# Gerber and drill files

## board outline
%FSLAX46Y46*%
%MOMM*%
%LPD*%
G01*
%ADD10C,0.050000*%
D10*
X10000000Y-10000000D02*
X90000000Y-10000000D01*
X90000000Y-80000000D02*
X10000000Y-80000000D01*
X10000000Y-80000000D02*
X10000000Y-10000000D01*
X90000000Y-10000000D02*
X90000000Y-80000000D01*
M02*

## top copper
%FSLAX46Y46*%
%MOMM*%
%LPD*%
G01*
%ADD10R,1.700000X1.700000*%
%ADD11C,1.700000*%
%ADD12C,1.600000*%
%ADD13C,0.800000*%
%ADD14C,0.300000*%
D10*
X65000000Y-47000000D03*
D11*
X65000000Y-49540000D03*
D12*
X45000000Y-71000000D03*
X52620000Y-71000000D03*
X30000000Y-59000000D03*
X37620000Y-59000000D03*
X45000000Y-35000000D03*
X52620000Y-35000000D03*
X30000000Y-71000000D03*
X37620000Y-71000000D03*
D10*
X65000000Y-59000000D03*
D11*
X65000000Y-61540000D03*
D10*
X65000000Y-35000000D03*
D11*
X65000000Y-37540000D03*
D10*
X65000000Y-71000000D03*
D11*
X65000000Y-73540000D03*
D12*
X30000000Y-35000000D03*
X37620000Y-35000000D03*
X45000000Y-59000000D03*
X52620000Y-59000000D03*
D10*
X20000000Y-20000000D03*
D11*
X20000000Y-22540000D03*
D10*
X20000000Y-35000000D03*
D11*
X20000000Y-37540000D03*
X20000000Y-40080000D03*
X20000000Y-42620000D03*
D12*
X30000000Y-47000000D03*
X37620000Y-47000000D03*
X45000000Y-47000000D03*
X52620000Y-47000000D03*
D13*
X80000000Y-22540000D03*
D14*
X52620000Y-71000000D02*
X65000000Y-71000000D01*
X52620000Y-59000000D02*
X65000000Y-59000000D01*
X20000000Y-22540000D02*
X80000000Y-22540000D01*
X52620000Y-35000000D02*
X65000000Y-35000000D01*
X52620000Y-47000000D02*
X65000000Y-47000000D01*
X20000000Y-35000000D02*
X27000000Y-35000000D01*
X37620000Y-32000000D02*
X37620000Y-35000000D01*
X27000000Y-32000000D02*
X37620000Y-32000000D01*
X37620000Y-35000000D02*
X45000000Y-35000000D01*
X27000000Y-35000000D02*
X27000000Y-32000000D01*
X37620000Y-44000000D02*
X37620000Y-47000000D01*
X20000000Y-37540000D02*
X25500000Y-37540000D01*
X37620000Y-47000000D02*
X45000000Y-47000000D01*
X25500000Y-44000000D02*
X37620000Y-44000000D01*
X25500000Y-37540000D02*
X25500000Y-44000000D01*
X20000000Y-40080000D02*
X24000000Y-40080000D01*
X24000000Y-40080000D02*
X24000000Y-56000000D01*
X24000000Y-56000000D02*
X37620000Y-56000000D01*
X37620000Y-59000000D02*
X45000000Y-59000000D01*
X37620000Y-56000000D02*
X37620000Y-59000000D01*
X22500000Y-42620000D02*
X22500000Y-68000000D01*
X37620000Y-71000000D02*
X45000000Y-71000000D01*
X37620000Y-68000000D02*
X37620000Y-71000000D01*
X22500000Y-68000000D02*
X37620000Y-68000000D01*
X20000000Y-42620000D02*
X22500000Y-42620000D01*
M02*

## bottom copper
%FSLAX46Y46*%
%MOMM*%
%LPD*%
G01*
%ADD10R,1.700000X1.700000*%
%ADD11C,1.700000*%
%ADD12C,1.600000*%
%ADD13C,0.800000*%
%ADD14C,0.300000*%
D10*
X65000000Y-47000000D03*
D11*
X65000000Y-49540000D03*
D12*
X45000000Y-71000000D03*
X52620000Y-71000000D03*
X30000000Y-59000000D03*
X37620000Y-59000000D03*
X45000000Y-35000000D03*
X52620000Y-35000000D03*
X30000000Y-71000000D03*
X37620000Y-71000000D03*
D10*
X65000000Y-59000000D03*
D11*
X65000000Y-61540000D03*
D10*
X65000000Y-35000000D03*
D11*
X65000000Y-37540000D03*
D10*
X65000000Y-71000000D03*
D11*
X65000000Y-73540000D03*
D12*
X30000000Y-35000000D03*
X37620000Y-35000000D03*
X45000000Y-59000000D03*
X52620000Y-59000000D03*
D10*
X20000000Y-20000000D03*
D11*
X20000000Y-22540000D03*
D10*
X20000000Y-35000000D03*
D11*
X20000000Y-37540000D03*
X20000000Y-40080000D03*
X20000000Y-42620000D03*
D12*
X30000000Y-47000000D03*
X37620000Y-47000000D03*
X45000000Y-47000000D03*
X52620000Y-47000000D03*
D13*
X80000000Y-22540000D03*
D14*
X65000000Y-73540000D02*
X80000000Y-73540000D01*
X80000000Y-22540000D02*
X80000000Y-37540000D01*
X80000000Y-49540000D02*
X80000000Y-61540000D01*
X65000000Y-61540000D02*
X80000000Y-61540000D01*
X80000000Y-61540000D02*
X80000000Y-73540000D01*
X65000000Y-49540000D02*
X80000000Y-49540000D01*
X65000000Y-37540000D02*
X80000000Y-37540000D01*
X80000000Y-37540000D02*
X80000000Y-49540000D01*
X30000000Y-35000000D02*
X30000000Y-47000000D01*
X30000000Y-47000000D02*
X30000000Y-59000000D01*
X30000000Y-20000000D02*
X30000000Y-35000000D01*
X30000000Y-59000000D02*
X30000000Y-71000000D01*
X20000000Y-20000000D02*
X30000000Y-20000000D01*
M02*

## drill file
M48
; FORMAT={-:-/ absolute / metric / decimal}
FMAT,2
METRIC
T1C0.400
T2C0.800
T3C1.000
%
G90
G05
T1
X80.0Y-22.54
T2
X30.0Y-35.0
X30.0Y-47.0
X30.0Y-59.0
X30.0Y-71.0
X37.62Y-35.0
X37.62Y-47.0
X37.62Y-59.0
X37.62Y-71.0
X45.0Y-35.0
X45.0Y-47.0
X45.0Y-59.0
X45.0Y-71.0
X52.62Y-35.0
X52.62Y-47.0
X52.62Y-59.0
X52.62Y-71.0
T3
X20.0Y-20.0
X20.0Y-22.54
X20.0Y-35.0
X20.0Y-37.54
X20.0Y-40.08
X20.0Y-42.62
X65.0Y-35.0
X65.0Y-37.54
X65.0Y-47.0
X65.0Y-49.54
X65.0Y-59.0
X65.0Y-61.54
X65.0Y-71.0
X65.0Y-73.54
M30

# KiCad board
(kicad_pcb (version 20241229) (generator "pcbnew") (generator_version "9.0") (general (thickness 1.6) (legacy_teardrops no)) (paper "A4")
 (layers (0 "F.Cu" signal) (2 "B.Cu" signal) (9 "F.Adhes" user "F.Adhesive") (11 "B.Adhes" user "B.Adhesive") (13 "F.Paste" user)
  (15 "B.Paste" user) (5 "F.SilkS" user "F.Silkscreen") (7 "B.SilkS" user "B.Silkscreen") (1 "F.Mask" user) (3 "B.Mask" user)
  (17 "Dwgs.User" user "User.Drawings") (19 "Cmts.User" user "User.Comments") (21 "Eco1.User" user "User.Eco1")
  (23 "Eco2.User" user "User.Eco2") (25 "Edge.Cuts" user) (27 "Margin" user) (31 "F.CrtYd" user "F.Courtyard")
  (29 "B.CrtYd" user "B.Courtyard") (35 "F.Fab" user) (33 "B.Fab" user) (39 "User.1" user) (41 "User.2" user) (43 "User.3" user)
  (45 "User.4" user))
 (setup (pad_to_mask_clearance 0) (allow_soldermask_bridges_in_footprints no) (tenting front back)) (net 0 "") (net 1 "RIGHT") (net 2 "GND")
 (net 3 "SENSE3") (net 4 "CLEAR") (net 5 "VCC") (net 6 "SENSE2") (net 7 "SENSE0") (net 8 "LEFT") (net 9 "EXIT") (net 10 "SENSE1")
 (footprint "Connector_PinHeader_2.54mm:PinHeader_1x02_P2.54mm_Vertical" (layer "F.Cu") (at 65 47)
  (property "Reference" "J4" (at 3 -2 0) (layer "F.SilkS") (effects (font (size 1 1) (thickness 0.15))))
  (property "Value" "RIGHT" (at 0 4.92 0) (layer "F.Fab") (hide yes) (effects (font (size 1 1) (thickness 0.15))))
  (pad "1" thru_hole rect (at 0 0) (size 1.7 1.7) (drill 1) (layers "*.Cu" "*.Mask") (remove_unused_layers no) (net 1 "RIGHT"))
  (pad "2" thru_hole circle (at 0 2.54) (size 1.7 1.7) (drill 1) (layers "*.Cu" "*.Mask") (remove_unused_layers no) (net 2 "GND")))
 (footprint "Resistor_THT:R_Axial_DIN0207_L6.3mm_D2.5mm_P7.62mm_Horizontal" (layer "F.Cu") (at 45 71)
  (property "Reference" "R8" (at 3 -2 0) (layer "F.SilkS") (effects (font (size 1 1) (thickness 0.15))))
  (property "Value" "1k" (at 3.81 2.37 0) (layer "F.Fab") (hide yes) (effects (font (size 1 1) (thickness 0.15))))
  (pad "1" thru_hole circle (at 0 0) (size 1.6 1.6) (drill 0.8) (layers "*.Cu" "*.Mask") (remove_unused_layers no) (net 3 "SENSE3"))
  (pad "2" thru_hole circle (at 7.62 0) (size 1.6 1.6) (drill 0.8) (layers "*.Cu" "*.Mask") (remove_unused_layers no) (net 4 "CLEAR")))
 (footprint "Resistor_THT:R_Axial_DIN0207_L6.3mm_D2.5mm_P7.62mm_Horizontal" (layer "F.Cu") (at 30 59)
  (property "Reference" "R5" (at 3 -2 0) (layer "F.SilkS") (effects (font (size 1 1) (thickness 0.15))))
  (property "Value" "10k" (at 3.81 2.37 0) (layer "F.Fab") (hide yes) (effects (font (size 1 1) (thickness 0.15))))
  (pad "1" thru_hole circle (at 0 0) (size 1.6 1.6) (drill 0.8) (layers "*.Cu" "*.Mask") (remove_unused_layers no) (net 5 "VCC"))
  (pad "2" thru_hole circle (at 7.62 0) (size 1.6 1.6) (drill 0.8) (layers "*.Cu" "*.Mask") (remove_unused_layers no) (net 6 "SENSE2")))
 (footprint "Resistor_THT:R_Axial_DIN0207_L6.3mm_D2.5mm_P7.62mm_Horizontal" (layer "F.Cu") (at 45 35)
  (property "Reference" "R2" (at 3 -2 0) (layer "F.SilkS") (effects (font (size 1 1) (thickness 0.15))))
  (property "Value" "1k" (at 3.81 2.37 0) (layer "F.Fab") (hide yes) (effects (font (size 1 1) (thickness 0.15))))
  (pad "1" thru_hole circle (at 0 0) (size 1.6 1.6) (drill 0.8) (layers "*.Cu" "*.Mask") (remove_unused_layers no) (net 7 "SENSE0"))
  (pad "2" thru_hole circle (at 7.62 0) (size 1.6 1.6) (drill 0.8) (layers "*.Cu" "*.Mask") (remove_unused_layers no) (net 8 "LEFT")))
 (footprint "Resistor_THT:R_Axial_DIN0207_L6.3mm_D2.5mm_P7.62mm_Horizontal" (layer "F.Cu") (at 30 71)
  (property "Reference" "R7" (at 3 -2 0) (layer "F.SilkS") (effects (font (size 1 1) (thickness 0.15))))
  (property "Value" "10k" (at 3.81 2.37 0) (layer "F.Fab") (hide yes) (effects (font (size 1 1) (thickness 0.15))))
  (pad "1" thru_hole circle (at 0 0) (size 1.6 1.6) (drill 0.8) (layers "*.Cu" "*.Mask") (remove_unused_layers no) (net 5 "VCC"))
  (pad "2" thru_hole circle (at 7.62 0) (size 1.6 1.6) (drill 0.8) (layers "*.Cu" "*.Mask") (remove_unused_layers no) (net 3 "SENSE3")))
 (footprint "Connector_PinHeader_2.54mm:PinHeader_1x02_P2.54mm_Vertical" (layer "F.Cu") (at 65 59)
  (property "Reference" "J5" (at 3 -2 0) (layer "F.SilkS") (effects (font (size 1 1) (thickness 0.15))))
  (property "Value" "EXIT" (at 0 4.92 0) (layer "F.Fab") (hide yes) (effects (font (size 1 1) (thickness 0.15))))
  (pad "1" thru_hole rect (at 0 0) (size 1.7 1.7) (drill 1) (layers "*.Cu" "*.Mask") (remove_unused_layers no) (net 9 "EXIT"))
  (pad "2" thru_hole circle (at 0 2.54) (size 1.7 1.7) (drill 1) (layers "*.Cu" "*.Mask") (remove_unused_layers no) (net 2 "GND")))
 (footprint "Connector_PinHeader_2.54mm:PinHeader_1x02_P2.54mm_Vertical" (layer "F.Cu") (at 65 35)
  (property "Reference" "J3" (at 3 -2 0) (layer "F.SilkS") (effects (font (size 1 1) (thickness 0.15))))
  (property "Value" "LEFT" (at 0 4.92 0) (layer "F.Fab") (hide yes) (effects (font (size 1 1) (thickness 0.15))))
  (pad "1" thru_hole rect (at 0 0) (size 1.7 1.7) (drill 1) (layers "*.Cu" "*.Mask") (remove_unused_layers no) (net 8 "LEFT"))
  (pad "2" thru_hole circle (at 0 2.54) (size 1.7 1.7) (drill 1) (layers "*.Cu" "*.Mask") (remove_unused_layers no) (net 2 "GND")))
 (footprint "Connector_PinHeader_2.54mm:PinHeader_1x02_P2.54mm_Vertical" (layer "F.Cu") (at 65 71)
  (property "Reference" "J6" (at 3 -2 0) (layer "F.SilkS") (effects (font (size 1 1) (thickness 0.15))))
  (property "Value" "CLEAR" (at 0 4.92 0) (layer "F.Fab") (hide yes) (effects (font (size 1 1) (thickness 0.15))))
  (pad "1" thru_hole rect (at 0 0) (size 1.7 1.7) (drill 1) (layers "*.Cu" "*.Mask") (remove_unused_layers no) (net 4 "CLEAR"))
  (pad "2" thru_hole circle (at 0 2.54) (size 1.7 1.7) (drill 1) (layers "*.Cu" "*.Mask") (remove_unused_layers no) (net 2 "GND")))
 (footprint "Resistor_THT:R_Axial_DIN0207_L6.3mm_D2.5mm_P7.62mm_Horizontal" (layer "F.Cu") (at 30 35)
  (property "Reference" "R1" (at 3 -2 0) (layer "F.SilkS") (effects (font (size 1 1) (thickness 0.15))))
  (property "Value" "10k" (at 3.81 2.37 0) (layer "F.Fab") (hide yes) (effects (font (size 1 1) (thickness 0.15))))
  (pad "1" thru_hole circle (at 0 0) (size 1.6 1.6) (drill 0.8) (layers "*.Cu" "*.Mask") (remove_unused_layers no) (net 5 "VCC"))
  (pad "2" thru_hole circle (at 7.62 0) (size 1.6 1.6) (drill 0.8) (layers "*.Cu" "*.Mask") (remove_unused_layers no) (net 7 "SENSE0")))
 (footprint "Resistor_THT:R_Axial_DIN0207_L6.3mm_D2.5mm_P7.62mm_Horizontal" (layer "F.Cu") (at 45 59)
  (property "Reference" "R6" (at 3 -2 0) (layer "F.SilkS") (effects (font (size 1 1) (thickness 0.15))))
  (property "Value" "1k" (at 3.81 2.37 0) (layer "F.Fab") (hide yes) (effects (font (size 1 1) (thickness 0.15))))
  (pad "1" thru_hole circle (at 0 0) (size 1.6 1.6) (drill 0.8) (layers "*.Cu" "*.Mask") (remove_unused_layers no) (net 6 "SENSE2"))
  (pad "2" thru_hole circle (at 7.62 0) (size 1.6 1.6) (drill 0.8) (layers "*.Cu" "*.Mask") (remove_unused_layers no) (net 9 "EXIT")))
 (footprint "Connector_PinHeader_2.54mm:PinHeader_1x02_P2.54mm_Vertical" (layer "F.Cu") (at 20 20)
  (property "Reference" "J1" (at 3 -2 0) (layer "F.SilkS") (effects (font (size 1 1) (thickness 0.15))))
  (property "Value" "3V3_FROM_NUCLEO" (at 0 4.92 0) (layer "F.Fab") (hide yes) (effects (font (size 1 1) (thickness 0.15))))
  (pad "1" thru_hole rect (at 0 0) (size 1.7 1.7) (drill 1) (layers "*.Cu" "*.Mask") (remove_unused_layers no) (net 5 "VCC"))
  (pad "2" thru_hole circle (at 0 2.54) (size 1.7 1.7) (drill 1) (layers "*.Cu" "*.Mask") (remove_unused_layers no) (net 2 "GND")))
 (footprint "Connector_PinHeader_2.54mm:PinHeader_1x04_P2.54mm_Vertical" (layer "F.Cu") (at 20 35)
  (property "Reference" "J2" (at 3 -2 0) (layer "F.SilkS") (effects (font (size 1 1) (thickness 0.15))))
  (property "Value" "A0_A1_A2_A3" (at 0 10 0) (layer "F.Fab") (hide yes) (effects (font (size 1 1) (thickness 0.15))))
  (pad "1" thru_hole rect (at 0 0) (size 1.7 1.7) (drill 1) (layers "*.Cu" "*.Mask") (remove_unused_layers no) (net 7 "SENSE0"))
  (pad "2" thru_hole circle (at 0 2.54) (size 1.7 1.7) (drill 1) (layers "*.Cu" "*.Mask") (remove_unused_layers no) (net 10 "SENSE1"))
  (pad "3" thru_hole circle (at 0 5.08) (size 1.7 1.7) (drill 1) (layers "*.Cu" "*.Mask") (remove_unused_layers no) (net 6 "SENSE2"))
  (pad "4" thru_hole circle (at 0 7.62) (size 1.7 1.7) (drill 1) (layers "*.Cu" "*.Mask") (remove_unused_layers no) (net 3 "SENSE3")))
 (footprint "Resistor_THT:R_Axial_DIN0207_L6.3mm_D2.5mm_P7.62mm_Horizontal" (layer "F.Cu") (at 30 47)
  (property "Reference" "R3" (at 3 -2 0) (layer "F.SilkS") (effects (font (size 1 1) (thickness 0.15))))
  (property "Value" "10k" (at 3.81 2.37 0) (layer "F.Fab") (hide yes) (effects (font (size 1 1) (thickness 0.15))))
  (pad "1" thru_hole circle (at 0 0) (size 1.6 1.6) (drill 0.8) (layers "*.Cu" "*.Mask") (remove_unused_layers no) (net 5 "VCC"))
  (pad "2" thru_hole circle (at 7.62 0) (size 1.6 1.6) (drill 0.8) (layers "*.Cu" "*.Mask") (remove_unused_layers no) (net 10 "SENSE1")))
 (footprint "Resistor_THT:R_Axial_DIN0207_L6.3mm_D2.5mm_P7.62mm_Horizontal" (layer "F.Cu") (at 45 47)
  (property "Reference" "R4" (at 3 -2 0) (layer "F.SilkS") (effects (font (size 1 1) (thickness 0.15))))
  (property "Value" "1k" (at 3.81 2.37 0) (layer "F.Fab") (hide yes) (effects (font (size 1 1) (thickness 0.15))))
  (pad "1" thru_hole circle (at 0 0) (size 1.6 1.6) (drill 0.8) (layers "*.Cu" "*.Mask") (remove_unused_layers no) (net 10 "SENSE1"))
  (pad "2" thru_hole circle (at 7.62 0) (size 1.6 1.6) (drill 0.8) (layers "*.Cu" "*.Mask") (remove_unused_layers no) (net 1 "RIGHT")))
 (gr_line (start 10 10) (end 90 10) (stroke (width 0.05) (type default)) (layer "Edge.Cuts"))
 (gr_line (start 90 80) (end 10 80) (stroke (width 0.05) (type default)) (layer "Edge.Cuts"))
 (gr_line (start 10 80) (end 10 10) (stroke (width 0.05) (type default)) (layer "Edge.Cuts"))
 (gr_line (start 90 10) (end 90 80) (stroke (width 0.05) (type default)) (layer "Edge.Cuts"))
 (segment (start 52.62 71) (end 65 71) (width 0.3) (layer "F.Cu") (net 4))
 (segment (start 52.62 59) (end 65 59) (width 0.3) (layer "F.Cu") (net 9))
 (segment (start 20 22.54) (end 80 22.54) (width 0.3) (layer "F.Cu") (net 2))
 (via (at 80 22.54) (size 0.8) (drill 0.4) (layers "F.Cu" "B.Cu") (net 2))
 (segment (start 65 73.54) (end 80 73.54) (width 0.3) (layer "B.Cu") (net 2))
 (segment (start 80 22.54) (end 80 37.54) (width 0.3) (layer "B.Cu") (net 2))
 (segment (start 80 49.54) (end 80 61.54) (width 0.3) (layer "B.Cu") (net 2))
 (segment (start 65 61.54) (end 80 61.54) (width 0.3) (layer "B.Cu") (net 2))
 (segment (start 80 61.54) (end 80 73.54) (width 0.3) (layer "B.Cu") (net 2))
 (segment (start 65 49.54) (end 80 49.54) (width 0.3) (layer "B.Cu") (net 2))
 (segment (start 65 37.54) (end 80 37.54) (width 0.3) (layer "B.Cu") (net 2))
 (segment (start 80 37.54) (end 80 49.54) (width 0.3) (layer "B.Cu") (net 2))
 (segment (start 52.62 35) (end 65 35) (width 0.3) (layer "F.Cu") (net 8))
 (segment (start 52.62 47) (end 65 47) (width 0.3) (layer "F.Cu") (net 1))
 (segment (start 20 35) (end 27 35) (width 0.3) (layer "F.Cu") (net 7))
 (segment (start 37.62 32) (end 37.62 35) (width 0.3) (layer "F.Cu") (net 7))
 (segment (start 27 32) (end 37.62 32) (width 0.3) (layer "F.Cu") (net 7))
 (segment (start 37.62 35) (end 45 35) (width 0.3) (layer "F.Cu") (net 7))
 (segment (start 27 35) (end 27 32) (width 0.3) (layer "F.Cu") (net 7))
 (segment (start 37.62 44) (end 37.62 47) (width 0.3) (layer "F.Cu") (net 10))
 (segment (start 20 37.54) (end 25.5 37.54) (width 0.3) (layer "F.Cu") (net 10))
 (segment (start 37.62 47) (end 45 47) (width 0.3) (layer "F.Cu") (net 10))
 (segment (start 25.5 44) (end 37.62 44) (width 0.3) (layer "F.Cu") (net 10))
 (segment (start 25.5 37.54) (end 25.5 44) (width 0.3) (layer "F.Cu") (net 10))
 (segment (start 20 40.08) (end 24 40.08) (width 0.3) (layer "F.Cu") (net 6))
 (segment (start 24 40.08) (end 24 56) (width 0.3) (layer "F.Cu") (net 6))
 (segment (start 24 56) (end 37.62 56) (width 0.3) (layer "F.Cu") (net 6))
 (segment (start 37.62 59) (end 45 59) (width 0.3) (layer "F.Cu") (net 6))
 (segment (start 37.62 56) (end 37.62 59) (width 0.3) (layer "F.Cu") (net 6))
 (segment (start 22.5 42.62) (end 22.5 68) (width 0.3) (layer "F.Cu") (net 3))
 (segment (start 37.62 71) (end 45 71) (width 0.3) (layer "F.Cu") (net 3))
 (segment (start 37.62 68) (end 37.62 71) (width 0.3) (layer "F.Cu") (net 3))
 (segment (start 22.5 68) (end 37.62 68) (width 0.3) (layer "F.Cu") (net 3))
 (segment (start 20 42.62) (end 22.5 42.62) (width 0.3) (layer "F.Cu") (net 3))
 (segment (start 30 35) (end 30 47) (width 0.3) (layer "B.Cu") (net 5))
 (segment (start 30 47) (end 30 59) (width 0.3) (layer "B.Cu") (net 5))
 (segment (start 30 20) (end 30 35) (width 0.3) (layer "B.Cu") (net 5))
 (segment (start 30 59) (end 30 71) (width 0.3) (layer "B.Cu") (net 5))
 (segment (start 20 20) (end 30 20) (width 0.3) (layer "B.Cu") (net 5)))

